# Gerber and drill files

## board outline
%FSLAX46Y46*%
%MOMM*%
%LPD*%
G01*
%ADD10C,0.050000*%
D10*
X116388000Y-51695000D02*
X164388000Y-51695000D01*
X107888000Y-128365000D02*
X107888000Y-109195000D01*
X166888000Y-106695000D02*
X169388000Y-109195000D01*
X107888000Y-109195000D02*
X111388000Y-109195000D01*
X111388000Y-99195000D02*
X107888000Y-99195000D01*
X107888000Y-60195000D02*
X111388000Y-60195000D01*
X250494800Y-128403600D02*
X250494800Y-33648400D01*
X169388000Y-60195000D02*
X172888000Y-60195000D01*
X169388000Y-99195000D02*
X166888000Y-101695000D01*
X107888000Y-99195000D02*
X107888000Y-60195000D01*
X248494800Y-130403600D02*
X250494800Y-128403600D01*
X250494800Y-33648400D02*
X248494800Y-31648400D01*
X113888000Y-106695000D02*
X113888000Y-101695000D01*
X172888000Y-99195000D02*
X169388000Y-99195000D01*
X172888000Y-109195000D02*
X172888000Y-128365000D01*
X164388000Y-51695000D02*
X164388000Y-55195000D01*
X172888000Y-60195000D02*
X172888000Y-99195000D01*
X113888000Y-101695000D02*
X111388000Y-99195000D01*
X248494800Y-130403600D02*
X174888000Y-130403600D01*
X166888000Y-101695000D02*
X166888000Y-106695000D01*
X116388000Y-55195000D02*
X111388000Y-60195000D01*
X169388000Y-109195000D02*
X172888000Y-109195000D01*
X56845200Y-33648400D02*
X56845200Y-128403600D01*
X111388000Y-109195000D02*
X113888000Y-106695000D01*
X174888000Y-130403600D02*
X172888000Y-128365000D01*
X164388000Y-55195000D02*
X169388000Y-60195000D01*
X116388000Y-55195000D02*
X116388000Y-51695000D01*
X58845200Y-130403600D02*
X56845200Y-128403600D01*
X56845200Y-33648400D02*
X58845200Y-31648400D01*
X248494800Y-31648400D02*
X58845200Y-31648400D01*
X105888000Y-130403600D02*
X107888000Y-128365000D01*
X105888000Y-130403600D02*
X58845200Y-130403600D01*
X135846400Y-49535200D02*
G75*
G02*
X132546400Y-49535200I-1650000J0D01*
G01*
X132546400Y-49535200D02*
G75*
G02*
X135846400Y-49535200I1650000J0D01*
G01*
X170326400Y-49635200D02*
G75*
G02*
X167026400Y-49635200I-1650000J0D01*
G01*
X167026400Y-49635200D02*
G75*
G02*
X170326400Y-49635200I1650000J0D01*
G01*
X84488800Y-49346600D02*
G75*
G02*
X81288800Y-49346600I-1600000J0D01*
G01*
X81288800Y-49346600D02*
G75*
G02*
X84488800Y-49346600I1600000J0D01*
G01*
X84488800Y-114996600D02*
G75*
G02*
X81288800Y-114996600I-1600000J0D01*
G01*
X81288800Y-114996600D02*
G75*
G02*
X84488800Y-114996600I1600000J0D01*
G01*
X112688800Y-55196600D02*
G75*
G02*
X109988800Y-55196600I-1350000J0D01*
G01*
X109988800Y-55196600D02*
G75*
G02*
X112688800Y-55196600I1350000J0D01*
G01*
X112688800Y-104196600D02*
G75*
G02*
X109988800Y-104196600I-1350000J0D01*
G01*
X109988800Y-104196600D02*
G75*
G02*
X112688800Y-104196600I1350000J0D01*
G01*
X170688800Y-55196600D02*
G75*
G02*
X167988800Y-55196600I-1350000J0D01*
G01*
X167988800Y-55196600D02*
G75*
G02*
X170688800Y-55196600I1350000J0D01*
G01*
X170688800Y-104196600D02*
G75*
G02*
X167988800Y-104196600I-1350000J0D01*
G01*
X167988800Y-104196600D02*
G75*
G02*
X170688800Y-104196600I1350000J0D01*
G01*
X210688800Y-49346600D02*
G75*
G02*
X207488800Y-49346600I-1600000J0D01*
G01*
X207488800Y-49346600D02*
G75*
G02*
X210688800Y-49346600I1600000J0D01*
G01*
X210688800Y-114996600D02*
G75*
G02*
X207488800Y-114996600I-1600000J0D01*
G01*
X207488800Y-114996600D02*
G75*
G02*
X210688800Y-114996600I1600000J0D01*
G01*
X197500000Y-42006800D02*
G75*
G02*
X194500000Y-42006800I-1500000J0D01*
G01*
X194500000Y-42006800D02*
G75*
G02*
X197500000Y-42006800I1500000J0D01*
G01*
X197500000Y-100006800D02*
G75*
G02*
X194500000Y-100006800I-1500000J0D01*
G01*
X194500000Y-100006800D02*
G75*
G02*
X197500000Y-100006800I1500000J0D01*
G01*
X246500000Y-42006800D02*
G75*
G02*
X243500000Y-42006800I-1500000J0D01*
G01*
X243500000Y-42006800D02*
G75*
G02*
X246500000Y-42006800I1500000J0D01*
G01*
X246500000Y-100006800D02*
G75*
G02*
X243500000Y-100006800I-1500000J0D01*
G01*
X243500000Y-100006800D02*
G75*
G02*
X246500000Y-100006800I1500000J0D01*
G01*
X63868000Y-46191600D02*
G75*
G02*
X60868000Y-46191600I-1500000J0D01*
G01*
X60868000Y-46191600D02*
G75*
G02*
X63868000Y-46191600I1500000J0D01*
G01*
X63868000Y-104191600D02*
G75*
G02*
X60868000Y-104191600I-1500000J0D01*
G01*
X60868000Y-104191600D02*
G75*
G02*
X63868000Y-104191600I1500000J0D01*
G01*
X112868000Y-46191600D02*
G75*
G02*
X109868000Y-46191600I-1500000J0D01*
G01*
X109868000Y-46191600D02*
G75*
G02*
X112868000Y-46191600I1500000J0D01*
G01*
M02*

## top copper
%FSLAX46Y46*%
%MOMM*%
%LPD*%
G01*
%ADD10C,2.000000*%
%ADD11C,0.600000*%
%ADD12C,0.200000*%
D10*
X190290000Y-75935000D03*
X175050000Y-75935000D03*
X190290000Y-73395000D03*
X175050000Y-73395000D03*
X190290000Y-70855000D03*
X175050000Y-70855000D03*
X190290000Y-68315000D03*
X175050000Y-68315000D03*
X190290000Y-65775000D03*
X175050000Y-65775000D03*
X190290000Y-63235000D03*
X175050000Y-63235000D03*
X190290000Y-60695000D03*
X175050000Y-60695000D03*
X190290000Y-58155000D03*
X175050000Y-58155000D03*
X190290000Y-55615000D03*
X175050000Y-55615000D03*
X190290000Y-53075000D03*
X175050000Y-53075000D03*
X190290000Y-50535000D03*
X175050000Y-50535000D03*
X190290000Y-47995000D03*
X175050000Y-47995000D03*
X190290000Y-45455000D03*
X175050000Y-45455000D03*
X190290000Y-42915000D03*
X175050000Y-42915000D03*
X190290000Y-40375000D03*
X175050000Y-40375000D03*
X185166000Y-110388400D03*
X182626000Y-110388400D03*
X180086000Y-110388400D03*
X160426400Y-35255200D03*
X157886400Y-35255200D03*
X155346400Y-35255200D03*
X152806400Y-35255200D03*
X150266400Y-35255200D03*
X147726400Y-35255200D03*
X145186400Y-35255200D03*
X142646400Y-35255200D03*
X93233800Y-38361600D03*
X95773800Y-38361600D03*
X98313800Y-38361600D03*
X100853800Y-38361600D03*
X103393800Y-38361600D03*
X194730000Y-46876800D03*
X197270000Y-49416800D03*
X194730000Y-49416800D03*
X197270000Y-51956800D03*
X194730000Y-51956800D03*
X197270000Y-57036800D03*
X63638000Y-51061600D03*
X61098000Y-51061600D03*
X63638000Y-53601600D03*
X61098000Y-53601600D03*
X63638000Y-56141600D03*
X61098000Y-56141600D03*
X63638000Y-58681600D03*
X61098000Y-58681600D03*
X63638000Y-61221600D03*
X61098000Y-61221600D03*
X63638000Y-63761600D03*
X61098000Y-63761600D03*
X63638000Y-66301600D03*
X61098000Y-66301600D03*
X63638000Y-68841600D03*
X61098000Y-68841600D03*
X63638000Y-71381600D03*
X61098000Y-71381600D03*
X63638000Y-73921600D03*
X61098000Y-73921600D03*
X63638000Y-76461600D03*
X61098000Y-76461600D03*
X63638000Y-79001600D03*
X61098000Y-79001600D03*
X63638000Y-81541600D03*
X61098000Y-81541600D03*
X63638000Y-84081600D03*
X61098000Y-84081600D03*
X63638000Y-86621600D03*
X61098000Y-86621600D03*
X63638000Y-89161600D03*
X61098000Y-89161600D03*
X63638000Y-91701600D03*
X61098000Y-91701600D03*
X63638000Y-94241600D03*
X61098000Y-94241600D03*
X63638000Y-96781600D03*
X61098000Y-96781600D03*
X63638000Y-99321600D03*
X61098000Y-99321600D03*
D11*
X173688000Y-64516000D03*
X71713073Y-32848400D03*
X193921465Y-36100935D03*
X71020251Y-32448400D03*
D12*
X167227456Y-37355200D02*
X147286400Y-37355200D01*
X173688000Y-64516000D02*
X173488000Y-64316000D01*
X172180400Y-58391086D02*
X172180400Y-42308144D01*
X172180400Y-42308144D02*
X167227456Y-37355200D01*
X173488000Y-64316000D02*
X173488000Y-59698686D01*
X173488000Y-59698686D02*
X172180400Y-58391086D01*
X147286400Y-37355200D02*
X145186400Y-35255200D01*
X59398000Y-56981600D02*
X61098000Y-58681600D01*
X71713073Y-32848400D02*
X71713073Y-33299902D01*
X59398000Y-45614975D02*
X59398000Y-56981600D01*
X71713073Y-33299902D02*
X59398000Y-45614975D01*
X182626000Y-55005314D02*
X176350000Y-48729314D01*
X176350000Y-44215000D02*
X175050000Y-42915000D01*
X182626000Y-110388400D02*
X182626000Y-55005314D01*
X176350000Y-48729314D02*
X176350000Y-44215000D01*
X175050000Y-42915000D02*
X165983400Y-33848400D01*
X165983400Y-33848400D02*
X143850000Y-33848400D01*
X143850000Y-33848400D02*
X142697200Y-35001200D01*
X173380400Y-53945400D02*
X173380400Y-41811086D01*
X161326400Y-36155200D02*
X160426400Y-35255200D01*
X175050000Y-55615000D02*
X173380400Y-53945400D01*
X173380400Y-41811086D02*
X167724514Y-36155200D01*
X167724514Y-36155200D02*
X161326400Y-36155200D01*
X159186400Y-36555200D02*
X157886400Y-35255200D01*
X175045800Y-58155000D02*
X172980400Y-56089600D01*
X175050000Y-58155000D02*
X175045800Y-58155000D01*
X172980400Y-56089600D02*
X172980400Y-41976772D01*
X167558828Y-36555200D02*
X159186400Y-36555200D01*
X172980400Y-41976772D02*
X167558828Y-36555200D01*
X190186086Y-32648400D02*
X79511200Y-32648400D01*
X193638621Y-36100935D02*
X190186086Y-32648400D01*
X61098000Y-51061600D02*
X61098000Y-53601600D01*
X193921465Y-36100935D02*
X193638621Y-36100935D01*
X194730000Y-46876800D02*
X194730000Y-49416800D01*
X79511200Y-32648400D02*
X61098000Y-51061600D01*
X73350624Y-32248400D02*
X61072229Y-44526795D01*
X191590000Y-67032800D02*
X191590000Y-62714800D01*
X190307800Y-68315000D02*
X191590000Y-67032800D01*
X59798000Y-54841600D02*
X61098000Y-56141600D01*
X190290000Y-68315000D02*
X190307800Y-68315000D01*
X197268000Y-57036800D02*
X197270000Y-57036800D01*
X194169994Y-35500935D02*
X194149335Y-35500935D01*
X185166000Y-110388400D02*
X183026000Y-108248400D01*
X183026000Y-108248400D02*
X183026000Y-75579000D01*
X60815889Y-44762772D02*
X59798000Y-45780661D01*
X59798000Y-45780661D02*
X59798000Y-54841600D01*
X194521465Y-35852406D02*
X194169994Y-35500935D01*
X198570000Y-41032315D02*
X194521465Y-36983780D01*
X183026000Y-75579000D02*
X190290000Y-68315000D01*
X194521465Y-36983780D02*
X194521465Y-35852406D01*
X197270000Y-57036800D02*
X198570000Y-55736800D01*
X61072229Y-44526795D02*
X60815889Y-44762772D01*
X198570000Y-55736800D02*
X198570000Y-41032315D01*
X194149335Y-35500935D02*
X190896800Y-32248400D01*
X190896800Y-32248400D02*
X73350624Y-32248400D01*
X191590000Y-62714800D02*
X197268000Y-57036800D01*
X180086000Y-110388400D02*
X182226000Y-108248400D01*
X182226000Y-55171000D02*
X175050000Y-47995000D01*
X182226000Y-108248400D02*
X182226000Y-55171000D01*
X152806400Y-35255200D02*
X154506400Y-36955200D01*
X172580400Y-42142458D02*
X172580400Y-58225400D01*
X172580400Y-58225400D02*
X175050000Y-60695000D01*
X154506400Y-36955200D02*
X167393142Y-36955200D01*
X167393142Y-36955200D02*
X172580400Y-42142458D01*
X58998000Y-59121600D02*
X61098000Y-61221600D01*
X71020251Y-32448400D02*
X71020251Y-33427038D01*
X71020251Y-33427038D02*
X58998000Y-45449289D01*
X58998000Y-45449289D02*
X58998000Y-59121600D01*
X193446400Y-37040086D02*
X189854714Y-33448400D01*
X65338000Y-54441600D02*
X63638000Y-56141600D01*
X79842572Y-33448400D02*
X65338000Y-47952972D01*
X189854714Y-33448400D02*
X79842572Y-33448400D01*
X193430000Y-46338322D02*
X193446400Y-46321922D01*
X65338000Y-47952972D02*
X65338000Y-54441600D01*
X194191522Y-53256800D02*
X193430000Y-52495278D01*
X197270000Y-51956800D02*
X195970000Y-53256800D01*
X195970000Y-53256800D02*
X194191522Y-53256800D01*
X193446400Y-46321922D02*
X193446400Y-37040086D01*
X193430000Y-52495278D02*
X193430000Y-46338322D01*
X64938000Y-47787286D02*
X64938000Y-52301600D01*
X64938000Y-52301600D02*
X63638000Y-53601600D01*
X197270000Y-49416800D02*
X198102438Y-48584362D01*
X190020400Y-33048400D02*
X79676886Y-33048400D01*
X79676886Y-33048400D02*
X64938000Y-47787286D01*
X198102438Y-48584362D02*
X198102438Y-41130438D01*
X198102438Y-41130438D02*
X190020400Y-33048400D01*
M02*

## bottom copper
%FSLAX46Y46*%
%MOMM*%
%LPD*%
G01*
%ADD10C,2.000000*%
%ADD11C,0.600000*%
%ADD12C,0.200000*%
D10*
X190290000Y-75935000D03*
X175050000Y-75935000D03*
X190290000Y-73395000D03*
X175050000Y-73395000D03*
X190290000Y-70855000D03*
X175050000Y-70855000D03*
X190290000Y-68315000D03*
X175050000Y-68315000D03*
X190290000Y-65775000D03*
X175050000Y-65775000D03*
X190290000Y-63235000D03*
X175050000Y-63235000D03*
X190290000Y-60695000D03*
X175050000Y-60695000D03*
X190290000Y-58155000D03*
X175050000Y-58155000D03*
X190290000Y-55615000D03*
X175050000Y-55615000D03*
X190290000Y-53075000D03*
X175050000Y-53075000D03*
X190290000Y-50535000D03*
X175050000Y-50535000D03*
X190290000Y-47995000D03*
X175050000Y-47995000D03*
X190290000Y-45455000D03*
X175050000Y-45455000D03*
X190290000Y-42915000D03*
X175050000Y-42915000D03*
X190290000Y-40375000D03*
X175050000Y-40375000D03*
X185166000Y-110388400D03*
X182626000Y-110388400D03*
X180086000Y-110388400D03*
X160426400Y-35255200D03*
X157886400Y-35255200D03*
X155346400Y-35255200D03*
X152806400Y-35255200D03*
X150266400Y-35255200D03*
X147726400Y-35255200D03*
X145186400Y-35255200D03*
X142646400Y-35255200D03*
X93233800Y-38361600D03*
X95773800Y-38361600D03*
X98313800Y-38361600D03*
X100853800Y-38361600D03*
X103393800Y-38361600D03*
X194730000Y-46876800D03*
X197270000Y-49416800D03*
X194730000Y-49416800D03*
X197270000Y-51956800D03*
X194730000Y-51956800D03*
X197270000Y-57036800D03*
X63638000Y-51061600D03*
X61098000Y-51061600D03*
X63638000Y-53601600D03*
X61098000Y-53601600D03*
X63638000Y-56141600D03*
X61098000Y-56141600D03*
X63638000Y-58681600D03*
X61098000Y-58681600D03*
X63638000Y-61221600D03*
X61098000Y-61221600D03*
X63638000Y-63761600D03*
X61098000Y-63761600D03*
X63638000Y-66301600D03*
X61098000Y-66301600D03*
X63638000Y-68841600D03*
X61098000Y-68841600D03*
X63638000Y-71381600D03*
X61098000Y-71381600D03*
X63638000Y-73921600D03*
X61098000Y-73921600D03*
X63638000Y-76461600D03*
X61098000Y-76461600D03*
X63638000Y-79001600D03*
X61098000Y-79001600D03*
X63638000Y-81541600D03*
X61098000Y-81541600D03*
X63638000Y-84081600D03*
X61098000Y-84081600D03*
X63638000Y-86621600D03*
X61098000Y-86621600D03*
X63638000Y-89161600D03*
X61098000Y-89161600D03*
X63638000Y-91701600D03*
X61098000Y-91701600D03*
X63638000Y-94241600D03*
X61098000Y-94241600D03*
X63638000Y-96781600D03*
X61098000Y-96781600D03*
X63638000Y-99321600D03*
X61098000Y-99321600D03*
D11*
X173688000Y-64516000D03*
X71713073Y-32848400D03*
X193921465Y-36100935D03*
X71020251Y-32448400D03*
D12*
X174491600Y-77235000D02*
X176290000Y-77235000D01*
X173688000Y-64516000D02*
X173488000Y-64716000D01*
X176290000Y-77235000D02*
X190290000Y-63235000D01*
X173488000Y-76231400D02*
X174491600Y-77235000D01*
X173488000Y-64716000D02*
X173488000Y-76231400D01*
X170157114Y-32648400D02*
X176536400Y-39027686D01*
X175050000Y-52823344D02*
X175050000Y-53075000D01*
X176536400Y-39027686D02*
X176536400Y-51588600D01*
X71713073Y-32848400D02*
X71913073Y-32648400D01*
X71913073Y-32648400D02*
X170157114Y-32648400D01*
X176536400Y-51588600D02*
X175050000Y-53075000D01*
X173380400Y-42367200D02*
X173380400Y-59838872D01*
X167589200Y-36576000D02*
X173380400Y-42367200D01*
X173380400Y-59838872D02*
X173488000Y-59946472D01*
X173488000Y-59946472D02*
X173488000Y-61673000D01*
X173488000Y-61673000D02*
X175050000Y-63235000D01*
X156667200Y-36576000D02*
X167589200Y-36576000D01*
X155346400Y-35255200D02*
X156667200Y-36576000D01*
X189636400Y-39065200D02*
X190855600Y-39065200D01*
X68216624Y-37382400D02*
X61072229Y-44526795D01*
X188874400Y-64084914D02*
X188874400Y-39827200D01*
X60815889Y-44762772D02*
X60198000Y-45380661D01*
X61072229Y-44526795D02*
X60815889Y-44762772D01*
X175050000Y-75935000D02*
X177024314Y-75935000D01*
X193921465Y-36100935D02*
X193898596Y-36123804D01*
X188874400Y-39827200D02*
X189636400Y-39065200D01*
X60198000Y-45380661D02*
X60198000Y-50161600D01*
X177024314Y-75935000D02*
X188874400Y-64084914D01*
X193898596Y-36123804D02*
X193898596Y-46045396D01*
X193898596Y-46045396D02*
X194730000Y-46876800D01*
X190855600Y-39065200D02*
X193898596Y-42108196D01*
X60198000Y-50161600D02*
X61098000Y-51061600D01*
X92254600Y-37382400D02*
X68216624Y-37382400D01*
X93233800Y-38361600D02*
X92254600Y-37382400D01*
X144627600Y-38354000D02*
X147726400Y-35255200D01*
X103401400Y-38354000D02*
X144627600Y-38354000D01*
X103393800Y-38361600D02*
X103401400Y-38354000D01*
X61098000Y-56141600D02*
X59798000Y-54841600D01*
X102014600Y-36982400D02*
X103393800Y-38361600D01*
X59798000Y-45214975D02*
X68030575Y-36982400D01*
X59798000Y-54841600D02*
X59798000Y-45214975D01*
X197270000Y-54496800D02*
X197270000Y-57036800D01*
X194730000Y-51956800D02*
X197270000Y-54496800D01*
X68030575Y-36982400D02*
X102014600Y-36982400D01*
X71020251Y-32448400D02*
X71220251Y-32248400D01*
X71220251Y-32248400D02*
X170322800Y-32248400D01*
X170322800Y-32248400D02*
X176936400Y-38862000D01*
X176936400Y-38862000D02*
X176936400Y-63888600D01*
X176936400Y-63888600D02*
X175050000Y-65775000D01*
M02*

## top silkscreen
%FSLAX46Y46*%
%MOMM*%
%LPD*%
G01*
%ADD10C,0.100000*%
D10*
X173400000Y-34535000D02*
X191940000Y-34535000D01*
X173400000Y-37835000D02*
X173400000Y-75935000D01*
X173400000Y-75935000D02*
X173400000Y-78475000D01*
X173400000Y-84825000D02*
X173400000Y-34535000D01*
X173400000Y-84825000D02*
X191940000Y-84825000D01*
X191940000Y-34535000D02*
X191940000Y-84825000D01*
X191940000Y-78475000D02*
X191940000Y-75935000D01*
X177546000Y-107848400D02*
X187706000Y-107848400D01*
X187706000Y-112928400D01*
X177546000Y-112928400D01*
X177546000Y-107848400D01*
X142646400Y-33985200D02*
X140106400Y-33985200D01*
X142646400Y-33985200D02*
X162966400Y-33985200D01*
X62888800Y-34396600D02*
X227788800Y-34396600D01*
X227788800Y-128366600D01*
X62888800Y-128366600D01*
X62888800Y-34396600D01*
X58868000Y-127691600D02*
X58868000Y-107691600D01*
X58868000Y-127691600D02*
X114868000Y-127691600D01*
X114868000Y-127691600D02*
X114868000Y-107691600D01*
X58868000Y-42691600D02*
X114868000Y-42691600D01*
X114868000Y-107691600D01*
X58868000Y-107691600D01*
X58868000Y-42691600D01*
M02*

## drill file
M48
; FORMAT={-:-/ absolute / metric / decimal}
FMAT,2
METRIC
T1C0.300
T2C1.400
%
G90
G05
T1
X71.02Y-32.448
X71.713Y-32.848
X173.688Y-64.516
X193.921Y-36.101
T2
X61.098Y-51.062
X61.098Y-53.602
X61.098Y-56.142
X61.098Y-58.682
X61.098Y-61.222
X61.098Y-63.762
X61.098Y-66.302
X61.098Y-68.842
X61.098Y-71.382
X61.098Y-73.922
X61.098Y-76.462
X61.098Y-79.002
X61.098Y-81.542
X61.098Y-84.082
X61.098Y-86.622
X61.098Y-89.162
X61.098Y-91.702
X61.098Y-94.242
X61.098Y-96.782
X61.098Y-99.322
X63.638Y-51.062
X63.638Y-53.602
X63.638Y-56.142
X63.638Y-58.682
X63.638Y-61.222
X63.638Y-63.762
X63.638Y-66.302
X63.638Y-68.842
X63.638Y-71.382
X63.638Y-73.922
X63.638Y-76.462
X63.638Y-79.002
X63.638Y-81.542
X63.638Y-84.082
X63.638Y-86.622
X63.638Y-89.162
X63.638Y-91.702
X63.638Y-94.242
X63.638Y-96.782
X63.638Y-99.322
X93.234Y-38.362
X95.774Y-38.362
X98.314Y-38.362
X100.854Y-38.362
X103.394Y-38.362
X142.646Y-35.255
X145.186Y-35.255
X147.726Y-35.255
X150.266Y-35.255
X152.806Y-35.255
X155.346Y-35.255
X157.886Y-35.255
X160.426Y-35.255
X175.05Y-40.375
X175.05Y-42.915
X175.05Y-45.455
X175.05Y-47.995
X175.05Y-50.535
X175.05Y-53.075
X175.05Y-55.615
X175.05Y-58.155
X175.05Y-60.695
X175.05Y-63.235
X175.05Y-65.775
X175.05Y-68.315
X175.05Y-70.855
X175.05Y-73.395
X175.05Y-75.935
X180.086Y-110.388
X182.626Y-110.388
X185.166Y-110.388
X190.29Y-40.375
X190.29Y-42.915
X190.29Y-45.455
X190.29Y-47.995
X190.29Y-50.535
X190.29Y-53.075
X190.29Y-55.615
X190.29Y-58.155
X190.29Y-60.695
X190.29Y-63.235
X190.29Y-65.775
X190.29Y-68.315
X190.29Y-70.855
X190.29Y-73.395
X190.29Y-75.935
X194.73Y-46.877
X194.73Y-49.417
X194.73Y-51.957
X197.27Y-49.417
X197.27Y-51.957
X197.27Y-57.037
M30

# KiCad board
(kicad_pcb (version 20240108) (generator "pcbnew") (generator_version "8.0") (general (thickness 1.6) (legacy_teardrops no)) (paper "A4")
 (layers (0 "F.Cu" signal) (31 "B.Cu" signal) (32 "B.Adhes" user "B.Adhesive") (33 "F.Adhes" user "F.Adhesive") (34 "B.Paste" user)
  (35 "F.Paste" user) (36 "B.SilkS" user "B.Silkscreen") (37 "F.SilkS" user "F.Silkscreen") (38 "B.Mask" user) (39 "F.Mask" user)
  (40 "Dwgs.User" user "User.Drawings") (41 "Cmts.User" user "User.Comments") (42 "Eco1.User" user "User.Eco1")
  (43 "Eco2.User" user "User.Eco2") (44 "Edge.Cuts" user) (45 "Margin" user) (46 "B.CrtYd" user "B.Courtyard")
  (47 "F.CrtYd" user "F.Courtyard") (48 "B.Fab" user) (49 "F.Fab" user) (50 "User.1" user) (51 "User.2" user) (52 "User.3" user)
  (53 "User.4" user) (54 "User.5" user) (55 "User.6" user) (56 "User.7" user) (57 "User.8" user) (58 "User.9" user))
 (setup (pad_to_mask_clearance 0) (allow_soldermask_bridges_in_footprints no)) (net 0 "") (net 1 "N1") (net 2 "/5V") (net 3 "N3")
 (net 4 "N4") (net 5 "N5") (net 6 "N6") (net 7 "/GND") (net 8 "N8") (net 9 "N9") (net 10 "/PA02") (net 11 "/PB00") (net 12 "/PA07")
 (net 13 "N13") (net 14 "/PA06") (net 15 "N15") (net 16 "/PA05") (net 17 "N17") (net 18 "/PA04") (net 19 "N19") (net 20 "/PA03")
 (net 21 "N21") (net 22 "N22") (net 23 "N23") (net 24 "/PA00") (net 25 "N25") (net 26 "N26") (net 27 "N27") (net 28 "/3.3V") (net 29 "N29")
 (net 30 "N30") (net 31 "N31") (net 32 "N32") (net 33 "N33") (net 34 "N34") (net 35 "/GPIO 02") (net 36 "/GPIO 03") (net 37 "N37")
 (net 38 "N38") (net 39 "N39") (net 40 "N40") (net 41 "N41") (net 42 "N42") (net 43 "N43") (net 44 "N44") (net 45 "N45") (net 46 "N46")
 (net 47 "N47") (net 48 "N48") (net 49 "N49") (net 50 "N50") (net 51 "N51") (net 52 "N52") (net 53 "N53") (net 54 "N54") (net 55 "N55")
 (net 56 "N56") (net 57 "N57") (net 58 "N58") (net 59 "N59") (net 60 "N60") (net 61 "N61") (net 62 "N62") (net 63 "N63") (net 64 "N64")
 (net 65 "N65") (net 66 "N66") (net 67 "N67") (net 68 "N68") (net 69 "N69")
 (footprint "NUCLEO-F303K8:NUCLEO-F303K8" (layer "F.Cu") (at 194.1 88 180)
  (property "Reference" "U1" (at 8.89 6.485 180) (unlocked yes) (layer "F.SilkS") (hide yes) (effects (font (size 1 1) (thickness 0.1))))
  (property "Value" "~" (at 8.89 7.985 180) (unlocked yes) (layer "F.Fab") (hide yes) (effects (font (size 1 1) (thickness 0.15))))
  (fp_line (start 20.7 53.465) (end 2.16 53.465) (stroke (width 0.1) (type default)) (layer "F.SilkS"))
  (fp_line (start 20.7 50.165) (end 20.7 12.065) (stroke (width 0.1) (type default)) (layer "F.SilkS"))
  (fp_line (start 20.7 12.065) (end 20.7 9.525) (stroke (width 0.1) (type default)) (layer "F.SilkS"))
  (fp_line (start 20.7 3.175) (end 20.7 53.465) (stroke (width 0.1) (type default)) (layer "F.SilkS"))
  (fp_line (start 20.7 3.175) (end 2.16 3.175) (stroke (width 0.1) (type default)) (layer "F.SilkS"))
  (fp_line (start 2.16 53.465) (end 2.16 3.175) (stroke (width 0.1) (type default)) (layer "F.SilkS"))
  (fp_line (start 2.16 9.525) (end 2.16 12.065) (stroke (width 0.1) (type default)) (layer "F.SilkS"))
  (pad "1" thru_hole circle (at 3.81 12.065 180) (size 2 2) (drill 1.4) (layers "*.Cu" "*.Mask") (remove_unused_layers no) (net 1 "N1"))
  (pad "2" thru_hole circle (at 19.05 12.065 180) (size 2 2) (drill 1.4) (layers "*.Cu" "*.Mask") (remove_unused_layers no) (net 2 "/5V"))
  (pad "3" thru_hole circle (at 3.81 14.605 180) (size 2 2) (drill 1.4) (layers "*.Cu" "*.Mask") (remove_unused_layers no) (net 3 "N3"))
  (pad "4" thru_hole circle (at 19.05 14.605 180) (size 2 2) (drill 1.4) (layers "*.Cu" "*.Mask") (remove_unused_layers no) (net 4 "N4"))
  (pad "5" thru_hole circle (at 3.81 17.145 180) (size 2 2) (drill 1.4) (layers "*.Cu" "*.Mask") (remove_unused_layers no) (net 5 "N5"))
  (pad "6" thru_hole circle (at 19.05 17.145 180) (size 2 2) (drill 1.4) (layers "*.Cu" "*.Mask") (remove_unused_layers no) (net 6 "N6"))
  (pad "7" thru_hole circle (at 3.81 19.685 180) (size 2 2) (drill 1.4) (layers "*.Cu" "*.Mask") (remove_unused_layers no) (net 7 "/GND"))
  (pad "8" thru_hole circle (at 19.05 19.685 180) (size 2 2) (drill 1.4) (layers "*.Cu" "*.Mask") (remove_unused_layers no) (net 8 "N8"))
  (pad "9" thru_hole circle (at 3.81 22.225 180) (size 2 2) (drill 1.4) (layers "*.Cu" "*.Mask") (remove_unused_layers no) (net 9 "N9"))
  (pad "10" thru_hole circle (at 19.05 22.225 180) (size 2 2) (drill 1.4) (layers "*.Cu" "*.Mask") (remove_unused_layers no)
   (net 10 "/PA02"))
  (pad "11" thru_hole circle (at 3.81 24.765 180) (size 2 2) (drill 1.4) (layers "*.Cu" "*.Mask") (remove_unused_layers no) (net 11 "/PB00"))
  (pad "12" thru_hole circle (at 19.05 24.765 180) (size 2 2) (drill 1.4) (layers "*.Cu" "*.Mask") (remove_unused_layers no)
   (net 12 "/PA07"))
  (pad "13" thru_hole circle (at 3.81 27.305 180) (size 2 2) (drill 1.4) (layers "*.Cu" "*.Mask") (remove_unused_layers no) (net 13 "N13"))
  (pad "14" thru_hole circle (at 19.05 27.305 180) (size 2 2) (drill 1.4) (layers "*.Cu" "*.Mask") (remove_unused_layers no)
   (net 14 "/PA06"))
  (pad "15" thru_hole circle (at 3.81 29.845 180) (size 2 2) (drill 1.4) (layers "*.Cu" "*.Mask") (remove_unused_layers no) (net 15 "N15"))
  (pad "16" thru_hole circle (at 19.05 29.845 180) (size 2 2) (drill 1.4) (layers "*.Cu" "*.Mask") (remove_unused_layers no)
   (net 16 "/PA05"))
  (pad "17" thru_hole circle (at 3.81 32.385 180) (size 2 2) (drill 1.4) (layers "*.Cu" "*.Mask") (remove_unused_layers no) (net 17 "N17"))
  (pad "18" thru_hole circle (at 19.05 32.385 180) (size 2 2) (drill 1.4) (layers "*.Cu" "*.Mask") (remove_unused_layers no)
   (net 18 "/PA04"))
  (pad "19" thru_hole circle (at 3.81 34.925 180) (size 2 2) (drill 1.4) (layers "*.Cu" "*.Mask") (remove_unused_layers no) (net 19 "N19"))
  (pad "20" thru_hole circle (at 19.05 34.925 180) (size 2 2) (drill 1.4) (layers "*.Cu" "*.Mask") (remove_unused_layers no)
   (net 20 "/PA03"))
  (pad "21" thru_hole circle (at 3.81 37.465 180) (size 2 2) (drill 1.4) (layers "*.Cu" "*.Mask") (remove_unused_layers no) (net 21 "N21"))
  (pad "22" thru_hole circle (at 19.05 37.465 180) (size 2 2) (drill 1.4) (layers "*.Cu" "*.Mask") (remove_unused_layers no) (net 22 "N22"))
  (pad "23" thru_hole circle (at 3.81 40.005 180) (size 2 2) (drill 1.4) (layers "*.Cu" "*.Mask") (remove_unused_layers no) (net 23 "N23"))
  (pad "24" thru_hole circle (at 19.05 40.005 180) (size 2 2) (drill 1.4) (layers "*.Cu" "*.Mask") (remove_unused_layers no)
   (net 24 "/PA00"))
  (pad "25" thru_hole circle (at 3.81 42.545 180) (size 2 2) (drill 1.4) (layers "*.Cu" "*.Mask") (remove_unused_layers no) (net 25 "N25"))
  (pad "26" thru_hole circle (at 19.05 42.545 180) (size 2 2) (drill 1.4) (layers "*.Cu" "*.Mask") (remove_unused_layers no) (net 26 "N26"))
  (pad "27" thru_hole circle (at 3.81 45.085 180) (size 2 2) (drill 1.4) (layers "*.Cu" "*.Mask") (remove_unused_layers no) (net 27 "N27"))
  (pad "28" thru_hole circle (at 19.05 45.085 180) (size 2 2) (drill 1.4) (layers "*.Cu" "*.Mask") (remove_unused_layers no)
   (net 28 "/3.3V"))
  (pad "29" thru_hole circle (at 3.81 47.625 180) (size 2 2) (drill 1.4) (layers "*.Cu" "*.Mask") (remove_unused_layers no) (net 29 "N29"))
  (pad "30" thru_hole circle (at 19.05 47.625 180) (size 2 2) (drill 1.4) (layers "*.Cu" "*.Mask") (remove_unused_layers no) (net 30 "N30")))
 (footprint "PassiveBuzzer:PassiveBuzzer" (layer "F.Cu") (at 187.706 107.8484 -90)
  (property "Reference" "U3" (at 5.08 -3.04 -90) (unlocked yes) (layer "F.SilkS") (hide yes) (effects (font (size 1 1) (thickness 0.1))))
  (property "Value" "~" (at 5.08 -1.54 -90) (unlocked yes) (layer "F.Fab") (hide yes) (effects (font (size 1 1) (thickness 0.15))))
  (fp_rect (start 0 0) (end 5.08 10.16) (stroke (width 0.1) (type default)) (fill none) (layer "F.SilkS"))
  (pad "1" thru_hole circle (at 2.54 2.54 270) (size 2 2) (drill 1.4) (layers "*.Cu" "*.Mask") (remove_unused_layers no) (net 7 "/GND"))
  (pad "2" thru_hole circle (at 2.54 5.08 270) (size 2 2) (drill 1.4) (layers "*.Cu" "*.Mask") (remove_unused_layers no) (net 28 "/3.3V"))
  (pad "3" thru_hole circle (at 2.54 7.62 270) (size 2 2) (drill 1.4) (layers "*.Cu" "*.Mask") (remove_unused_layers no) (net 24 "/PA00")))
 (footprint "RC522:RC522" (layer "F.Cu") (at 162.9664 32.7152 -90)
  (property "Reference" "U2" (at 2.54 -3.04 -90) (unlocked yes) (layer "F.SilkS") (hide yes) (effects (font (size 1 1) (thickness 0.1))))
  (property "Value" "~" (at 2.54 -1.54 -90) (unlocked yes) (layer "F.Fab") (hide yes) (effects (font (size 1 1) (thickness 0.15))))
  (fp_line (start 1.27 20.32) (end 1.27 22.86) (stroke (width 0.1) (type default)) (layer "F.SilkS"))
  (fp_line (start 1.27 20.32) (end 1.27 0) (stroke (width 0.1) (type default)) (layer "F.SilkS"))
  (fp_circle (center 16.82 28.77) (end 18.47 28.77) (stroke (width 0.05) (type default)) (fill none) (layer "Edge.Cuts"))
  (fp_circle (center 16.92 -5.71) (end 18.57 -5.71) (stroke (width 0.05) (type default)) (fill none) (layer "Edge.Cuts"))
  (pad "1" thru_hole circle (at 2.54 2.54 270) (size 2 2) (drill 1.4) (layers "*.Cu" "*.Mask") (remove_unused_layers no) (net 18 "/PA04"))
  (pad "2" thru_hole circle (at 2.54 5.08 270) (size 2 2) (drill 1.4) (layers "*.Cu" "*.Mask") (remove_unused_layers no) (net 16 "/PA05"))
  (pad "3" thru_hole circle (at 2.54 7.62 270) (size 2 2) (drill 1.4) (layers "*.Cu" "*.Mask") (remove_unused_layers no) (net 12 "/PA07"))
  (pad "4" thru_hole circle (at 2.54 10.16 270) (size 2 2) (drill 1.4) (layers "*.Cu" "*.Mask") (remove_unused_layers no) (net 14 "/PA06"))
  (pad "5" thru_hole circle (at 2.54 12.7 270) (size 2 2) (drill 1.4) (layers "*.Cu" "*.Mask") (remove_unused_layers no) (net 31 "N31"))
  (pad "6" thru_hole circle (at 2.54 15.24 270) (size 2 2) (drill 1.4) (layers "*.Cu" "*.Mask") (remove_unused_layers no) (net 7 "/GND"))
  (pad "7" thru_hole circle (at 2.54 17.78 270) (size 2 2) (drill 1.4) (layers "*.Cu" "*.Mask") (remove_unused_layers no) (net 11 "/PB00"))
  (pad "8" thru_hole circle (at 2.54 20.32 270) (size 2 2) (drill 1.4) (layers "*.Cu" "*.Mask") (remove_unused_layers no) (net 28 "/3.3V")))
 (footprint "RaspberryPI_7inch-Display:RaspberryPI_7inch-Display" (layer "F.Cu") (at 107.8388 51.6966)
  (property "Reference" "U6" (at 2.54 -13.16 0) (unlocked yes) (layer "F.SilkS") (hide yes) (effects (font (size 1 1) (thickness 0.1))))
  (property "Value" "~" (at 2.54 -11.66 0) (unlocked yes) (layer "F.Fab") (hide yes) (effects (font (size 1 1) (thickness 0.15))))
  (fp_rect (start -44.95 -17.3) (end 119.95 76.67) (stroke (width 0.1) (type default)) (fill none) (layer "F.SilkS"))
  (fp_circle (center -24.95 -2.35) (end -23.35 -2.35) (stroke (width 0.05) (type default)) (fill none) (layer "Edge.Cuts"))
  (fp_circle (center -24.95 63.3) (end -23.35 63.3) (stroke (width 0.05) (type default)) (fill none) (layer "Edge.Cuts"))
  (fp_circle (center 3.5 3.5) (end 4.85 3.5) (stroke (width 0.05) (type default)) (fill none) (layer "Edge.Cuts"))
  (fp_circle (center 3.5 52.5) (end 4.85 52.5) (stroke (width 0.05) (type default)) (fill none) (layer "Edge.Cuts"))
  (fp_circle (center 61.5 3.5) (end 62.85 3.5) (stroke (width 0.05) (type default)) (fill none) (layer "Edge.Cuts"))
  (fp_circle (center 61.5 52.5) (end 62.85 52.5) (stroke (width 0.05) (type default)) (fill none) (layer "Edge.Cuts"))
  (fp_circle (center 101.25 -2.35) (end 102.85 -2.35) (stroke (width 0.05) (type default)) (fill none) (layer "Edge.Cuts"))
  (fp_circle (center 101.25 63.3) (end 102.85 63.3) (stroke (width 0.05) (type default)) (fill none) (layer "Edge.Cuts"))
  (pad "1" thru_hole circle (at -14.605 -13.335 90) (size 2 2) (drill 1.4) (layers "*.Cu" "*.Mask") (remove_unused_layers no) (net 2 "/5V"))
  (pad "2" thru_hole circle (at -12.065 -13.335 90) (size 2 2) (drill 1.4) (layers "*.Cu" "*.Mask") (remove_unused_layers no) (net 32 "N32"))
  (pad "3" thru_hole circle (at -9.525 -13.335 90) (size 2 2) (drill 1.4) (layers "*.Cu" "*.Mask") (remove_unused_layers no) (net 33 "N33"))
  (pad "4" thru_hole circle (at -6.985 -13.335 90) (size 2 2) (drill 1.4) (layers "*.Cu" "*.Mask") (remove_unused_layers no) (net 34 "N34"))
  (pad "5" thru_hole circle (at -4.445 -13.335 90) (size 2 2) (drill 1.4) (layers "*.Cu" "*.Mask") (remove_unused_layers no) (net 7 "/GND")))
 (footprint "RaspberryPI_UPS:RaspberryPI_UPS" (layer "B.Cu") (at 196 42 180)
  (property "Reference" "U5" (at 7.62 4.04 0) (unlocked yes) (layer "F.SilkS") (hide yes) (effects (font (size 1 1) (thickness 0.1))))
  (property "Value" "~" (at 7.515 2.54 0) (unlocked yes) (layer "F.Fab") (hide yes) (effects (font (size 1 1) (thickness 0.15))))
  (fp_circle (center 0 -0.0068) (end 1.5 -0.0068) (stroke (width 0.05) (type solid)) (fill none) (layer "Edge.Cuts"))
  (fp_circle (center 0 -58.0068) (end 1.5 -58.0068) (stroke (width 0.05) (type default)) (fill none) (layer "Edge.Cuts"))
  (fp_circle (center -49 -0.0068) (end -47.5 -0.0068) (stroke (width 0.05) (type default)) (fill none) (layer "Edge.Cuts"))
  (fp_circle (center -49 -58.0068) (end -47.5 -58.0068) (stroke (width 0.05) (type default)) (fill none) (layer "Edge.Cuts"))
  (pad "1" thru_hole circle (at 1.27 -4.8768 180) (size 2 2) (drill 1.4) (layers "*.Cu" "*.Mask") (remove_unused_layers no) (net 2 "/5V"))
  (pad "2" thru_hole circle (at -1.27 -7.4168 180) (size 2 2) (drill 1.4) (layers "*.Cu" "*.Mask") (remove_unused_layers no)
   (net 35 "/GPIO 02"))
  (pad "3" thru_hole circle (at 1.27 -7.4168 180) (size 2 2) (drill 1.4) (layers "*.Cu" "*.Mask") (remove_unused_layers no) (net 2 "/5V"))
  (pad "4" thru_hole circle (at -1.27 -9.9568 180) (size 2 2) (drill 1.4) (layers "*.Cu" "*.Mask") (remove_unused_layers no)
   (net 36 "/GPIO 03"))
  (pad "5" thru_hole circle (at 1.27 -9.9568 180) (size 2 2) (drill 1.4) (layers "*.Cu" "*.Mask") (remove_unused_layers no) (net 7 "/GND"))
  (pad "6" thru_hole circle (at -1.27 -15.0368 180) (size 2 2) (drill 1.4) (layers "*.Cu" "*.Mask") (remove_unused_layers no) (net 7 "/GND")))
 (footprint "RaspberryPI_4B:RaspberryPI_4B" (layer "B.Cu") (at 60.568 78.7916 180)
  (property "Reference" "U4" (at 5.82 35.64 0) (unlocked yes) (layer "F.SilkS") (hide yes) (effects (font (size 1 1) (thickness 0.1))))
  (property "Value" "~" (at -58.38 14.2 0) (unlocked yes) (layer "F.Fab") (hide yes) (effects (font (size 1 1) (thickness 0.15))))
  (fp_line (start 1.7 -48.9) (end 1.7 -28.9) (stroke (width 0.1) (type default)) (layer "F.SilkS"))
  (fp_line (start 1.7 -48.9) (end -54.3 -48.9) (stroke (width 0.1) (type default)) (layer "F.SilkS"))
  (fp_line (start -54.3 -48.9) (end -54.3 -28.9) (stroke (width 0.1) (type default)) (layer "F.SilkS"))
  (fp_rect (start -54.3 36.1) (end 1.7 -28.9) (stroke (width 0.1) (type default)) (fill none) (layer "F.SilkS"))
  (fp_circle (center -1.8 32.6) (end -0.3 32.6) (stroke (width 0.05) (type default)) (fill none) (layer "Edge.Cuts"))
  (fp_circle (center -1.8 -25.4) (end -0.3 -25.4) (stroke (width 0.05) (type default)) (fill none) (layer "Edge.Cuts"))
  (fp_circle (center -50.8 32.6) (end -49.3 32.6) (stroke (width 0.05) (type default)) (fill none) (layer "Edge.Cuts"))
  (pad "1" thru_hole circle (at -3.07 27.73 180) (size 2 2) (drill 1.4) (layers "*.Cu" "*.Mask") (remove_unused_layers no) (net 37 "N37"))
  (pad "2" thru_hole circle (at -0.53 27.73 180) (size 2 2) (drill 1.4) (layers "*.Cu" "*.Mask") (remove_unused_layers no) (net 2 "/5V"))
  (pad "3" thru_hole circle (at -3.07 25.19 180) (size 2 2) (drill 1.4) (layers "*.Cu" "*.Mask") (remove_unused_layers no)
   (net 35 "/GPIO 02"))
  (pad "4" thru_hole circle (at -0.53 25.19 180) (size 2 2) (drill 1.4) (layers "*.Cu" "*.Mask") (remove_unused_layers no) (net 2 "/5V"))
  (pad "5" thru_hole circle (at -3.07 22.65 180) (size 2 2) (drill 1.4) (layers "*.Cu" "*.Mask") (remove_unused_layers no)
   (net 36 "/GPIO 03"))
  (pad "6" thru_hole circle (at -0.53 22.65 180) (size 2 2) (drill 1.4) (layers "*.Cu" "*.Mask") (remove_unused_layers no) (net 7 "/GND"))
  (pad "7" thru_hole circle (at -3.07 20.11 180) (size 2 2) (drill 1.4) (layers "*.Cu" "*.Mask") (remove_unused_layers no) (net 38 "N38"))
  (pad "8" thru_hole circle (at -0.53 20.11 180) (size 2 2) (drill 1.4) (layers "*.Cu" "*.Mask") (remove_unused_layers no) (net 20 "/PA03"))
  (pad "9" thru_hole circle (at -3.07 17.57 180) (size 2 2) (drill 1.4) (layers "*.Cu" "*.Mask") (remove_unused_layers no) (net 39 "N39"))
  (pad "10" thru_hole circle (at -0.53 17.57 180) (size 2 2) (drill 1.4) (layers "*.Cu" "*.Mask") (remove_unused_layers no) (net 10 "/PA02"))
  (pad "11" thru_hole circle (at -3.07 15.03 180) (size 2 2) (drill 1.4) (layers "*.Cu" "*.Mask") (remove_unused_layers no) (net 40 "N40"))
  (pad "12" thru_hole circle (at -0.53 15.03 180) (size 2 2) (drill 1.4) (layers "*.Cu" "*.Mask") (remove_unused_layers no) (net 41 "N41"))
  (pad "13" thru_hole circle (at -3.07 12.49 180) (size 2 2) (drill 1.4) (layers "*.Cu" "*.Mask") (remove_unused_layers no) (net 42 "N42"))
  (pad "14" thru_hole circle (at -0.53 12.49 180) (size 2 2) (drill 1.4) (layers "*.Cu" "*.Mask") (remove_unused_layers no) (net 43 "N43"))
  (pad "15" thru_hole circle (at -3.07 9.95 180) (size 2 2) (drill 1.4) (layers "*.Cu" "*.Mask") (remove_unused_layers no) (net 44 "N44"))
  (pad "16" thru_hole circle (at -0.53 9.95 180) (size 2 2) (drill 1.4) (layers "*.Cu" "*.Mask") (remove_unused_layers no) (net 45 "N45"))
  (pad "17" thru_hole circle (at -3.07 7.41 180) (size 2 2) (drill 1.4) (layers "*.Cu" "*.Mask") (remove_unused_layers no) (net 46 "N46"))
  (pad "18" thru_hole circle (at -0.53 7.41 180) (size 2 2) (drill 1.4) (layers "*.Cu" "*.Mask") (remove_unused_layers no) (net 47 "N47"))
  (pad "19" thru_hole circle (at -3.07 4.87 180) (size 2 2) (drill 1.4) (layers "*.Cu" "*.Mask") (remove_unused_layers no) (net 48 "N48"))
  (pad "20" thru_hole circle (at -0.53 4.87 180) (size 2 2) (drill 1.4) (layers "*.Cu" "*.Mask") (remove_unused_layers no) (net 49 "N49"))
  (pad "21" thru_hole circle (at -3.07 2.33 180) (size 2 2) (drill 1.4) (layers "*.Cu" "*.Mask") (remove_unused_layers no) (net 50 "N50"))
  (pad "22" thru_hole circle (at -0.53 2.33 180) (size 2 2) (drill 1.4) (layers "*.Cu" "*.Mask") (remove_unused_layers no) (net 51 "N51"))
  (pad "23" thru_hole circle (at -3.07 -0.21 180) (size 2 2) (drill 1.4) (layers "*.Cu" "*.Mask") (remove_unused_layers no) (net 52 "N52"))
  (pad "24" thru_hole circle (at -0.53 -0.21 180) (size 2 2) (drill 1.4) (layers "*.Cu" "*.Mask") (remove_unused_layers no) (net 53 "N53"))
  (pad "25" thru_hole circle (at -3.07 -2.75 180) (size 2 2) (drill 1.4) (layers "*.Cu" "*.Mask") (remove_unused_layers no) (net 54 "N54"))
  (pad "26" thru_hole circle (at -0.53 -2.75 180) (size 2 2) (drill 1.4) (layers "*.Cu" "*.Mask") (remove_unused_layers no) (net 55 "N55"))
  (pad "27" thru_hole circle (at -3.07 -5.29 180) (size 2 2) (drill 1.4) (layers "*.Cu" "*.Mask") (remove_unused_layers no) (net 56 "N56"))
  (pad "28" thru_hole circle (at -0.53 -5.29 180) (size 2 2) (drill 1.4) (layers "*.Cu" "*.Mask") (remove_unused_layers no) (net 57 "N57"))
  (pad "29" thru_hole circle (at -3.07 -7.83 180) (size 2 2) (drill 1.4) (layers "*.Cu" "*.Mask") (remove_unused_layers no) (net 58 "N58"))
  (pad "30" thru_hole circle (at -0.53 -7.83 180) (size 2 2) (drill 1.4) (layers "*.Cu" "*.Mask") (remove_unused_layers no) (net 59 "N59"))
  (pad "31" thru_hole circle (at -3.07 -10.37 180) (size 2 2) (drill 1.4) (layers "*.Cu" "*.Mask") (remove_unused_layers no) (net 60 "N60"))
  (pad "32" thru_hole circle (at -0.53 -10.37 180) (size 2 2) (drill 1.4) (layers "*.Cu" "*.Mask") (remove_unused_layers no) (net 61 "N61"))
  (pad "33" thru_hole circle (at -3.07 -12.91 180) (size 2 2) (drill 1.4) (layers "*.Cu" "*.Mask") (remove_unused_layers no) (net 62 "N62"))
  (pad "34" thru_hole circle (at -0.53 -12.91 180) (size 2 2) (drill 1.4) (layers "*.Cu" "*.Mask") (remove_unused_layers no) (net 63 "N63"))
  (pad "35" thru_hole circle (at -3.07 -15.45 180) (size 2 2) (drill 1.4) (layers "*.Cu" "*.Mask") (remove_unused_layers no) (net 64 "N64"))
  (pad "36" thru_hole circle (at -0.53 -15.45 180) (size 2 2) (drill 1.4) (layers "*.Cu" "*.Mask") (remove_unused_layers no) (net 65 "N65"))
  (pad "37" thru_hole circle (at -3.07 -17.99 180) (size 2 2) (drill 1.4) (layers "*.Cu" "*.Mask") (remove_unused_layers no) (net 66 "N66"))
  (pad "38" thru_hole circle (at -0.53 -17.99 180) (size 2 2) (drill 1.4) (layers "*.Cu" "*.Mask") (remove_unused_layers no) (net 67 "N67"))
  (pad "39" thru_hole circle (at -3.07 -20.53 180) (size 2 2) (drill 1.4) (layers "*.Cu" "*.Mask") (remove_unused_layers no) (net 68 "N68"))
  (pad "40" thru_hole circle (at -0.53 -20.53 180) (size 2 2) (drill 1.4) (layers "*.Cu" "*.Mask") (remove_unused_layers no) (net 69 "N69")))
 (gr_line (start 116.388 51.695) (end 164.388 51.695) (stroke (width 0.05) (type default)) (layer "Edge.Cuts"))
 (gr_line (start 107.888 128.365) (end 107.888 109.195) (stroke (width 0.05) (type default)) (layer "Edge.Cuts"))
 (gr_line (start 166.888 106.695) (end 169.388 109.195) (stroke (width 0.05) (type default)) (layer "Edge.Cuts"))
 (gr_line (start 107.888 109.195) (end 111.388 109.195) (stroke (width 0.05) (type default)) (layer "Edge.Cuts"))
 (gr_line (start 111.388 99.195) (end 107.888 99.195) (stroke (width 0.05) (type default)) (layer "Edge.Cuts"))
 (gr_line (start 107.888 60.195) (end 111.388 60.195) (stroke (width 0.05) (type default)) (layer "Edge.Cuts"))
 (gr_line (start 250.4948 128.4036) (end 250.4948 33.6484) (stroke (width 0.05) (type default)) (layer "Edge.Cuts"))
 (gr_line (start 169.388 60.195) (end 172.888 60.195) (stroke (width 0.05) (type default)) (layer "Edge.Cuts"))
 (gr_line (start 169.388 99.195) (end 166.888 101.695) (stroke (width 0.05) (type default)) (layer "Edge.Cuts"))
 (gr_line (start 107.888 99.195) (end 107.888 60.195) (stroke (width 0.05) (type default)) (layer "Edge.Cuts"))
 (gr_line (start 248.4948 130.4036) (end 250.4948 128.4036) (stroke (width 0.05) (type default)) (layer "Edge.Cuts"))
 (gr_line (start 250.4948 33.6484) (end 248.4948 31.6484) (stroke (width 0.05) (type default)) (layer "Edge.Cuts"))
 (gr_line (start 113.888 106.695) (end 113.888 101.695) (stroke (width 0.05) (type default)) (layer "Edge.Cuts"))
 (gr_line (start 172.888 99.195) (end 169.388 99.195) (stroke (width 0.05) (type default)) (layer "Edge.Cuts"))
 (gr_line (start 172.888 109.195) (end 172.888 128.365) (stroke (width 0.05) (type default)) (layer "Edge.Cuts"))
 (gr_line (start 164.388 51.695) (end 164.388 55.195) (stroke (width 0.05) (type default)) (layer "Edge.Cuts"))
 (gr_line (start 172.888 60.195) (end 172.888 99.195) (stroke (width 0.05) (type default)) (layer "Edge.Cuts"))
 (gr_line (start 113.888 101.695) (end 111.388 99.195) (stroke (width 0.05) (type default)) (layer "Edge.Cuts"))
 (gr_line (start 248.4948 130.4036) (end 174.888 130.4036) (stroke (width 0.05) (type default)) (layer "Edge.Cuts"))
 (gr_line (start 166.888 101.695) (end 166.888 106.695) (stroke (width 0.05) (type default)) (layer "Edge.Cuts"))
 (gr_line (start 116.388 55.195) (end 111.388 60.195) (stroke (width 0.05) (type default)) (layer "Edge.Cuts"))
 (gr_line (start 169.388 109.195) (end 172.888 109.195) (stroke (width 0.05) (type default)) (layer "Edge.Cuts"))
 (gr_line (start 56.8452 33.6484) (end 56.8452 128.4036) (stroke (width 0.05) (type default)) (layer "Edge.Cuts"))
 (gr_line (start 111.388 109.195) (end 113.888 106.695) (stroke (width 0.05) (type default)) (layer "Edge.Cuts"))
 (gr_line (start 174.888 130.4036) (end 172.888 128.365) (stroke (width 0.05) (type default)) (layer "Edge.Cuts"))
 (gr_line (start 164.388 55.195) (end 169.388 60.195) (stroke (width 0.05) (type default)) (layer "Edge.Cuts"))
 (gr_line (start 116.388 55.195) (end 116.388 51.695) (stroke (width 0.05) (type default)) (layer "Edge.Cuts"))
 (gr_line (start 58.8452 130.4036) (end 56.8452 128.4036) (stroke (width 0.05) (type default)) (layer "Edge.Cuts"))
 (gr_line (start 56.8452 33.6484) (end 58.8452 31.6484) (stroke (width 0.05) (type default)) (layer "Edge.Cuts"))
 (gr_line (start 248.4948 31.6484) (end 58.8452 31.6484) (stroke (width 0.05) (type default)) (layer "Edge.Cuts"))
 (gr_line (start 105.888 130.4036) (end 107.888 128.365) (stroke (width 0.05) (type default)) (layer "Edge.Cuts"))
 (gr_line (start 105.888 130.4036) (end 58.8452 130.4036) (stroke (width 0.05) (type default)) (layer "Edge.Cuts"))
 (segment (start 167.227456 37.3552) (end 147.2864 37.3552) (width 0.2) (layer "F.Cu") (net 11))
 (segment (start 173.688 64.516) (end 173.488 64.316) (width 0.2) (layer "F.Cu") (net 11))
 (segment (start 172.1804 58.391086) (end 172.1804 42.308144) (width 0.2) (layer "F.Cu") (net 11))
 (segment (start 172.1804 42.308144) (end 167.227456 37.3552) (width 0.2) (layer "F.Cu") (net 11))
 (segment (start 173.488 64.316) (end 173.488 59.698686) (width 0.2) (layer "F.Cu") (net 11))
 (segment (start 173.488 59.698686) (end 172.1804 58.391086) (width 0.2) (layer "F.Cu") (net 11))
 (segment (start 147.2864 37.3552) (end 145.1864 35.2552) (width 0.2) (layer "F.Cu") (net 11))
 (via (at 173.688 64.516) (size 0.6) (drill 0.3) (layers "F.Cu" "B.Cu") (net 11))
 (segment (start 174.4916 77.235) (end 176.29 77.235) (width 0.2) (layer "B.Cu") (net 11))
 (segment (start 173.688 64.516) (end 173.488 64.716) (width 0.2) (layer "B.Cu") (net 11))
 (segment (start 176.29 77.235) (end 190.29 63.235) (width 0.2) (layer "B.Cu") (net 11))
 (segment (start 173.488 76.2314) (end 174.4916 77.235) (width 0.2) (layer "B.Cu") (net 11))
 (segment (start 173.488 64.716) (end 173.488 76.2314) (width 0.2) (layer "B.Cu") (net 11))
 (segment (start 59.398 56.9816) (end 61.098 58.6816) (width 0.2) (layer "F.Cu") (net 20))
 (segment (start 71.713073 32.8484) (end 71.713073 33.299902) (width 0.2) (layer "F.Cu") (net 20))
 (segment (start 59.398 45.614975) (end 59.398 56.9816) (width 0.2) (layer "F.Cu") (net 20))
 (segment (start 71.713073 33.299902) (end 59.398 45.614975) (width 0.2) (layer "F.Cu") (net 20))
 (via (at 71.713073 32.8484) (size 0.6) (drill 0.3) (layers "F.Cu" "B.Cu") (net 20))
 (segment (start 170.157114 32.6484) (end 176.5364 39.027686) (width 0.2) (layer "B.Cu") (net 20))
 (segment (start 175.05 52.823344) (end 175.05 53.075) (width 0.2) (layer "B.Cu") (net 20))
 (segment (start 176.5364 39.027686) (end 176.5364 51.5886) (width 0.2) (layer "B.Cu") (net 20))
 (segment (start 71.713073 32.8484) (end 71.913073 32.6484) (width 0.2) (layer "B.Cu") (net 20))
 (segment (start 71.913073 32.6484) (end 170.157114 32.6484) (width 0.2) (layer "B.Cu") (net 20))
 (segment (start 176.5364 51.5886) (end 175.05 53.075) (width 0.2) (layer "B.Cu") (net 20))
 (segment (start 182.626 55.005314) (end 176.35 48.729314) (width 0.2) (layer "F.Cu") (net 28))
 (segment (start 176.35 44.215) (end 175.05 42.915) (width 0.2) (layer "F.Cu") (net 28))
 (segment (start 182.626 110.3884) (end 182.626 55.005314) (width 0.2) (layer "F.Cu") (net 28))
 (segment (start 176.35 48.729314) (end 176.35 44.215) (width 0.2) (layer "F.Cu") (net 28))
 (segment (start 175.05 42.915) (end 165.9834 33.8484) (width 0.2) (layer "F.Cu") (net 28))
 (segment (start 165.9834 33.8484) (end 143.85 33.8484) (width 0.2) (layer "F.Cu") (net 28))
 (segment (start 143.85 33.8484) (end 142.6972 35.0012) (width 0.2) (layer "F.Cu") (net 28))
 (segment (start 173.3804 53.9454) (end 173.3804 41.811086) (width 0.2) (layer "F.Cu") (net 18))
 (segment (start 161.3264 36.1552) (end 160.4264 35.2552) (width 0.2) (layer "F.Cu") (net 18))
 (segment (start 175.05 55.615) (end 173.3804 53.9454) (width 0.2) (layer "F.Cu") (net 18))
 (segment (start 173.3804 41.811086) (end 167.724514 36.1552) (width 0.2) (layer "F.Cu") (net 18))
 (segment (start 167.724514 36.1552) (end 161.3264 36.1552) (width 0.2) (layer "F.Cu") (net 18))
 (segment (start 173.3804 42.3672) (end 173.3804 59.838872) (width 0.2) (layer "B.Cu") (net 12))
 (segment (start 167.5892 36.576) (end 173.3804 42.3672) (width 0.2) (layer "B.Cu") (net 12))
 (segment (start 173.3804 59.838872) (end 173.488 59.946472) (width 0.2) (layer "B.Cu") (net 12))
 (segment (start 173.488 59.946472) (end 173.488 61.673) (width 0.2) (layer "B.Cu") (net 12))
 (segment (start 173.488 61.673) (end 175.05 63.235) (width 0.2) (layer "B.Cu") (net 12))
 (segment (start 156.6672 36.576) (end 167.5892 36.576) (width 0.2) (layer "B.Cu") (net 12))
 (segment (start 155.3464 35.2552) (end 156.6672 36.576) (width 0.2) (layer "B.Cu") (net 12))
 (segment (start 159.1864 36.5552) (end 157.8864 35.2552) (width 0.2) (layer "F.Cu") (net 16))
 (segment (start 175.0458 58.155) (end 172.9804 56.0896) (width 0.2) (layer "F.Cu") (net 16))
 (segment (start 175.05 58.155) (end 175.0458 58.155) (width 0.2) (layer "F.Cu") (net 16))
 (segment (start 172.9804 56.0896) (end 172.9804 41.976772) (width 0.2) (layer "F.Cu") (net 16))
 (segment (start 167.558828 36.5552) (end 159.1864 36.5552) (width 0.2) (layer "F.Cu") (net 16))
 (segment (start 172.9804 41.976772) (end 167.558828 36.5552) (width 0.2) (layer "F.Cu") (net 16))
 (segment (start 190.186086 32.6484) (end 79.5112 32.6484) (width 0.2) (layer "F.Cu") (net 2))
 (segment (start 193.638621 36.100935) (end 190.186086 32.6484) (width 0.2) (layer "F.Cu") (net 2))
 (segment (start 61.098 51.0616) (end 61.098 53.6016) (width 0.2) (layer "F.Cu") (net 2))
 (segment (start 193.921465 36.100935) (end 193.638621 36.100935) (width 0.2) (layer "F.Cu") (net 2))
 (segment (start 194.73 46.8768) (end 194.73 49.4168) (width 0.2) (layer "F.Cu") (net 2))
 (segment (start 79.5112 32.6484) (end 61.098 51.0616) (width 0.2) (layer "F.Cu") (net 2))
 (via (at 193.921465 36.100935) (size 0.6) (drill 0.3) (layers "F.Cu" "B.Cu") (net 2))
 (segment (start 189.6364 39.0652) (end 190.8556 39.0652) (width 0.2) (layer "B.Cu") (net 2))
 (segment (start 68.216624 37.3824) (end 61.072229 44.526795) (width 0.2) (layer "B.Cu") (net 2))
 (segment (start 188.8744 64.084914) (end 188.8744 39.8272) (width 0.2) (layer "B.Cu") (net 2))
 (segment (start 60.815889 44.762772) (end 60.198 45.380661) (width 0.2) (layer "B.Cu") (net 2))
 (segment (start 61.072229 44.526795) (end 60.815889 44.762772) (width 0.2) (layer "B.Cu") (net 2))
 (segment (start 175.05 75.935) (end 177.024314 75.935) (width 0.2) (layer "B.Cu") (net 2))
 (segment (start 193.921465 36.100935) (end 193.898596 36.123804) (width 0.2) (layer "B.Cu") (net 2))
 (segment (start 188.8744 39.8272) (end 189.6364 39.0652) (width 0.2) (layer "B.Cu") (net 2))
 (segment (start 60.198 45.380661) (end 60.198 50.1616) (width 0.2) (layer "B.Cu") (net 2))
 (segment (start 177.024314 75.935) (end 188.8744 64.084914) (width 0.2) (layer "B.Cu") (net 2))
 (segment (start 193.898596 36.123804) (end 193.898596 46.045396) (width 0.2) (layer "B.Cu") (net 2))
 (segment (start 193.898596 46.045396) (end 194.73 46.8768) (width 0.2) (layer "B.Cu") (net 2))
 (segment (start 190.8556 39.0652) (end 193.898596 42.108196) (width 0.2) (layer "B.Cu") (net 2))
 (segment (start 60.198 50.1616) (end 61.098 51.0616) (width 0.2) (layer "B.Cu") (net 2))
 (segment (start 92.2546 37.3824) (end 68.216624 37.3824) (width 0.2) (layer "B.Cu") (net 2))
 (segment (start 93.2338 38.3616) (end 92.2546 37.3824) (width 0.2) (layer "B.Cu") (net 2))
 (segment (start 73.350624 32.2484) (end 61.072229 44.526795) (width 0.2) (layer "F.Cu") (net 7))
 (segment (start 191.59 67.0328) (end 191.59 62.7148) (width 0.2) (layer "F.Cu") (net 7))
 (segment (start 190.3078 68.315) (end 191.59 67.0328) (width 0.2) (layer "F.Cu") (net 7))
 (segment (start 59.798 54.8416) (end 61.098 56.1416) (width 0.2) (layer "F.Cu") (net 7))
 (segment (start 190.29 68.315) (end 190.3078 68.315) (width 0.2) (layer "F.Cu") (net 7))
 (segment (start 197.268 57.0368) (end 197.27 57.0368) (width 0.2) (layer "F.Cu") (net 7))
 (segment (start 194.169994 35.500935) (end 194.149335 35.500935) (width 0.2) (layer "F.Cu") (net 7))
 (segment (start 185.166 110.3884) (end 183.026 108.2484) (width 0.2) (layer "F.Cu") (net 7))
 (segment (start 183.026 108.2484) (end 183.026 75.579) (width 0.2) (layer "F.Cu") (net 7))
 (segment (start 60.815889 44.762772) (end 59.798 45.780661) (width 0.2) (layer "F.Cu") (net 7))
 (segment (start 59.798 45.780661) (end 59.798 54.8416) (width 0.2) (layer "F.Cu") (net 7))
 (segment (start 194.521465 35.852406) (end 194.169994 35.500935) (width 0.2) (layer "F.Cu") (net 7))
 (segment (start 198.57 41.032315) (end 194.521465 36.98378) (width 0.2) (layer "F.Cu") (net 7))
 (segment (start 183.026 75.579) (end 190.29 68.315) (width 0.2) (layer "F.Cu") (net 7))
 (segment (start 194.521465 36.98378) (end 194.521465 35.852406) (width 0.2) (layer "F.Cu") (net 7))
 (segment (start 197.27 57.0368) (end 198.57 55.7368) (width 0.2) (layer "F.Cu") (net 7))
 (segment (start 61.072229 44.526795) (end 60.815889 44.762772) (width 0.2) (layer "F.Cu") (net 7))
 (segment (start 198.57 55.7368) (end 198.57 41.032315) (width 0.2) (layer "F.Cu") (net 7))
 (segment (start 194.149335 35.500935) (end 190.8968 32.2484) (width 0.2) (layer "F.Cu") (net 7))
 (segment (start 190.8968 32.2484) (end 73.350624 32.2484) (width 0.2) (layer "F.Cu") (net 7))
 (segment (start 191.59 62.7148) (end 197.268 57.0368) (width 0.2) (layer "F.Cu") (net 7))
 (segment (start 144.6276 38.354) (end 147.7264 35.2552) (width 0.2) (layer "B.Cu") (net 7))
 (segment (start 103.4014 38.354) (end 144.6276 38.354) (width 0.2) (layer "B.Cu") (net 7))
 (segment (start 103.3938 38.3616) (end 103.4014 38.354) (width 0.2) (layer "B.Cu") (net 7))
 (segment (start 61.098 56.1416) (end 59.798 54.8416) (width 0.2) (layer "B.Cu") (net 7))
 (segment (start 102.0146 36.9824) (end 103.3938 38.3616) (width 0.2) (layer "B.Cu") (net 7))
 (segment (start 59.798 45.214975) (end 68.030575 36.9824) (width 0.2) (layer "B.Cu") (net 7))
 (segment (start 59.798 54.8416) (end 59.798 45.214975) (width 0.2) (layer "B.Cu") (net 7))
 (segment (start 197.27 54.4968) (end 197.27 57.0368) (width 0.2) (layer "B.Cu") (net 7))
 (segment (start 194.73 51.9568) (end 197.27 54.4968) (width 0.2) (layer "B.Cu") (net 7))
 (segment (start 68.030575 36.9824) (end 102.0146 36.9824) (width 0.2) (layer "B.Cu") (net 7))
 (segment (start 180.086 110.3884) (end 182.226 108.2484) (width 0.2) (layer "F.Cu") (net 24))
 (segment (start 182.226 55.171) (end 175.05 47.995) (width 0.2) (layer "F.Cu") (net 24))
 (segment (start 182.226 108.2484) (end 182.226 55.171) (width 0.2) (layer "F.Cu") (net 24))
 (segment (start 152.8064 35.2552) (end 154.5064 36.9552) (width 0.2) (layer "F.Cu") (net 14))
 (segment (start 172.5804 42.142458) (end 172.5804 58.2254) (width 0.2) (layer "F.Cu") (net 14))
 (segment (start 172.5804 58.2254) (end 175.05 60.695) (width 0.2) (layer "F.Cu") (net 14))
 (segment (start 154.5064 36.9552) (end 167.393142 36.9552) (width 0.2) (layer "F.Cu") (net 14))
 (segment (start 167.393142 36.9552) (end 172.5804 42.142458) (width 0.2) (layer "F.Cu") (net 14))
 (segment (start 58.998 59.1216) (end 61.098 61.2216) (width 0.2) (layer "F.Cu") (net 10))
 (segment (start 71.020251 32.4484) (end 71.020251 33.427038) (width 0.2) (layer "F.Cu") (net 10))
 (segment (start 71.020251 33.427038) (end 58.998 45.449289) (width 0.2) (layer "F.Cu") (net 10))
 (segment (start 58.998 45.449289) (end 58.998 59.1216) (width 0.2) (layer "F.Cu") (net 10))
 (via (at 71.020251 32.4484) (size 0.6) (drill 0.3) (layers "F.Cu" "B.Cu") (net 10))
 (segment (start 71.020251 32.4484) (end 71.220251 32.2484) (width 0.2) (layer "B.Cu") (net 10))
 (segment (start 71.220251 32.2484) (end 170.3228 32.2484) (width 0.2) (layer "B.Cu") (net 10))
 (segment (start 170.3228 32.2484) (end 176.9364 38.862) (width 0.2) (layer "B.Cu") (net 10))
 (segment (start 176.9364 38.862) (end 176.9364 63.8886) (width 0.2) (layer "B.Cu") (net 10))
 (segment (start 176.9364 63.8886) (end 175.05 65.775) (width 0.2) (layer "B.Cu") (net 10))
 (segment (start 193.4464 37.040086) (end 189.854714 33.4484) (width 0.2) (layer "F.Cu") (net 36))
 (segment (start 65.338 54.4416) (end 63.638 56.1416) (width 0.2) (layer "F.Cu") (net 36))
 (segment (start 79.842572 33.4484) (end 65.338 47.952972) (width 0.2) (layer "F.Cu") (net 36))
 (segment (start 189.854714 33.4484) (end 79.842572 33.4484) (width 0.2) (layer "F.Cu") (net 36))
 (segment (start 193.43 46.338322) (end 193.4464 46.321922) (width 0.2) (layer "F.Cu") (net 36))
 (segment (start 65.338 47.952972) (end 65.338 54.4416) (width 0.2) (layer "F.Cu") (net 36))
 (segment (start 194.191522 53.2568) (end 193.43 52.495278) (width 0.2) (layer "F.Cu") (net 36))
 (segment (start 197.27 51.9568) (end 195.97 53.2568) (width 0.2) (layer "F.Cu") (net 36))
 (segment (start 195.97 53.2568) (end 194.191522 53.2568) (width 0.2) (layer "F.Cu") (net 36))
 (segment (start 193.4464 46.321922) (end 193.4464 37.040086) (width 0.2) (layer "F.Cu") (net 36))
 (segment (start 193.43 52.495278) (end 193.43 46.338322) (width 0.2) (layer "F.Cu") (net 36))
 (segment (start 64.938 47.787286) (end 64.938 52.3016) (width 0.2) (layer "F.Cu") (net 35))
 (segment (start 64.938 52.3016) (end 63.638 53.6016) (width 0.2) (layer "F.Cu") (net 35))
 (segment (start 197.27 49.4168) (end 198.102438 48.584362) (width 0.2) (layer "F.Cu") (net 35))
 (segment (start 190.0204 33.0484) (end 79.676886 33.0484) (width 0.2) (layer "F.Cu") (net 35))
 (segment (start 79.676886 33.0484) (end 64.938 47.787286) (width 0.2) (layer "F.Cu") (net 35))
 (segment (start 198.102438 48.584362) (end 198.102438 41.130438) (width 0.2) (layer "F.Cu") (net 35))
 (segment (start 198.102438 41.130438) (end 190.0204 33.0484) (width 0.2) (layer "F.Cu") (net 35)))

